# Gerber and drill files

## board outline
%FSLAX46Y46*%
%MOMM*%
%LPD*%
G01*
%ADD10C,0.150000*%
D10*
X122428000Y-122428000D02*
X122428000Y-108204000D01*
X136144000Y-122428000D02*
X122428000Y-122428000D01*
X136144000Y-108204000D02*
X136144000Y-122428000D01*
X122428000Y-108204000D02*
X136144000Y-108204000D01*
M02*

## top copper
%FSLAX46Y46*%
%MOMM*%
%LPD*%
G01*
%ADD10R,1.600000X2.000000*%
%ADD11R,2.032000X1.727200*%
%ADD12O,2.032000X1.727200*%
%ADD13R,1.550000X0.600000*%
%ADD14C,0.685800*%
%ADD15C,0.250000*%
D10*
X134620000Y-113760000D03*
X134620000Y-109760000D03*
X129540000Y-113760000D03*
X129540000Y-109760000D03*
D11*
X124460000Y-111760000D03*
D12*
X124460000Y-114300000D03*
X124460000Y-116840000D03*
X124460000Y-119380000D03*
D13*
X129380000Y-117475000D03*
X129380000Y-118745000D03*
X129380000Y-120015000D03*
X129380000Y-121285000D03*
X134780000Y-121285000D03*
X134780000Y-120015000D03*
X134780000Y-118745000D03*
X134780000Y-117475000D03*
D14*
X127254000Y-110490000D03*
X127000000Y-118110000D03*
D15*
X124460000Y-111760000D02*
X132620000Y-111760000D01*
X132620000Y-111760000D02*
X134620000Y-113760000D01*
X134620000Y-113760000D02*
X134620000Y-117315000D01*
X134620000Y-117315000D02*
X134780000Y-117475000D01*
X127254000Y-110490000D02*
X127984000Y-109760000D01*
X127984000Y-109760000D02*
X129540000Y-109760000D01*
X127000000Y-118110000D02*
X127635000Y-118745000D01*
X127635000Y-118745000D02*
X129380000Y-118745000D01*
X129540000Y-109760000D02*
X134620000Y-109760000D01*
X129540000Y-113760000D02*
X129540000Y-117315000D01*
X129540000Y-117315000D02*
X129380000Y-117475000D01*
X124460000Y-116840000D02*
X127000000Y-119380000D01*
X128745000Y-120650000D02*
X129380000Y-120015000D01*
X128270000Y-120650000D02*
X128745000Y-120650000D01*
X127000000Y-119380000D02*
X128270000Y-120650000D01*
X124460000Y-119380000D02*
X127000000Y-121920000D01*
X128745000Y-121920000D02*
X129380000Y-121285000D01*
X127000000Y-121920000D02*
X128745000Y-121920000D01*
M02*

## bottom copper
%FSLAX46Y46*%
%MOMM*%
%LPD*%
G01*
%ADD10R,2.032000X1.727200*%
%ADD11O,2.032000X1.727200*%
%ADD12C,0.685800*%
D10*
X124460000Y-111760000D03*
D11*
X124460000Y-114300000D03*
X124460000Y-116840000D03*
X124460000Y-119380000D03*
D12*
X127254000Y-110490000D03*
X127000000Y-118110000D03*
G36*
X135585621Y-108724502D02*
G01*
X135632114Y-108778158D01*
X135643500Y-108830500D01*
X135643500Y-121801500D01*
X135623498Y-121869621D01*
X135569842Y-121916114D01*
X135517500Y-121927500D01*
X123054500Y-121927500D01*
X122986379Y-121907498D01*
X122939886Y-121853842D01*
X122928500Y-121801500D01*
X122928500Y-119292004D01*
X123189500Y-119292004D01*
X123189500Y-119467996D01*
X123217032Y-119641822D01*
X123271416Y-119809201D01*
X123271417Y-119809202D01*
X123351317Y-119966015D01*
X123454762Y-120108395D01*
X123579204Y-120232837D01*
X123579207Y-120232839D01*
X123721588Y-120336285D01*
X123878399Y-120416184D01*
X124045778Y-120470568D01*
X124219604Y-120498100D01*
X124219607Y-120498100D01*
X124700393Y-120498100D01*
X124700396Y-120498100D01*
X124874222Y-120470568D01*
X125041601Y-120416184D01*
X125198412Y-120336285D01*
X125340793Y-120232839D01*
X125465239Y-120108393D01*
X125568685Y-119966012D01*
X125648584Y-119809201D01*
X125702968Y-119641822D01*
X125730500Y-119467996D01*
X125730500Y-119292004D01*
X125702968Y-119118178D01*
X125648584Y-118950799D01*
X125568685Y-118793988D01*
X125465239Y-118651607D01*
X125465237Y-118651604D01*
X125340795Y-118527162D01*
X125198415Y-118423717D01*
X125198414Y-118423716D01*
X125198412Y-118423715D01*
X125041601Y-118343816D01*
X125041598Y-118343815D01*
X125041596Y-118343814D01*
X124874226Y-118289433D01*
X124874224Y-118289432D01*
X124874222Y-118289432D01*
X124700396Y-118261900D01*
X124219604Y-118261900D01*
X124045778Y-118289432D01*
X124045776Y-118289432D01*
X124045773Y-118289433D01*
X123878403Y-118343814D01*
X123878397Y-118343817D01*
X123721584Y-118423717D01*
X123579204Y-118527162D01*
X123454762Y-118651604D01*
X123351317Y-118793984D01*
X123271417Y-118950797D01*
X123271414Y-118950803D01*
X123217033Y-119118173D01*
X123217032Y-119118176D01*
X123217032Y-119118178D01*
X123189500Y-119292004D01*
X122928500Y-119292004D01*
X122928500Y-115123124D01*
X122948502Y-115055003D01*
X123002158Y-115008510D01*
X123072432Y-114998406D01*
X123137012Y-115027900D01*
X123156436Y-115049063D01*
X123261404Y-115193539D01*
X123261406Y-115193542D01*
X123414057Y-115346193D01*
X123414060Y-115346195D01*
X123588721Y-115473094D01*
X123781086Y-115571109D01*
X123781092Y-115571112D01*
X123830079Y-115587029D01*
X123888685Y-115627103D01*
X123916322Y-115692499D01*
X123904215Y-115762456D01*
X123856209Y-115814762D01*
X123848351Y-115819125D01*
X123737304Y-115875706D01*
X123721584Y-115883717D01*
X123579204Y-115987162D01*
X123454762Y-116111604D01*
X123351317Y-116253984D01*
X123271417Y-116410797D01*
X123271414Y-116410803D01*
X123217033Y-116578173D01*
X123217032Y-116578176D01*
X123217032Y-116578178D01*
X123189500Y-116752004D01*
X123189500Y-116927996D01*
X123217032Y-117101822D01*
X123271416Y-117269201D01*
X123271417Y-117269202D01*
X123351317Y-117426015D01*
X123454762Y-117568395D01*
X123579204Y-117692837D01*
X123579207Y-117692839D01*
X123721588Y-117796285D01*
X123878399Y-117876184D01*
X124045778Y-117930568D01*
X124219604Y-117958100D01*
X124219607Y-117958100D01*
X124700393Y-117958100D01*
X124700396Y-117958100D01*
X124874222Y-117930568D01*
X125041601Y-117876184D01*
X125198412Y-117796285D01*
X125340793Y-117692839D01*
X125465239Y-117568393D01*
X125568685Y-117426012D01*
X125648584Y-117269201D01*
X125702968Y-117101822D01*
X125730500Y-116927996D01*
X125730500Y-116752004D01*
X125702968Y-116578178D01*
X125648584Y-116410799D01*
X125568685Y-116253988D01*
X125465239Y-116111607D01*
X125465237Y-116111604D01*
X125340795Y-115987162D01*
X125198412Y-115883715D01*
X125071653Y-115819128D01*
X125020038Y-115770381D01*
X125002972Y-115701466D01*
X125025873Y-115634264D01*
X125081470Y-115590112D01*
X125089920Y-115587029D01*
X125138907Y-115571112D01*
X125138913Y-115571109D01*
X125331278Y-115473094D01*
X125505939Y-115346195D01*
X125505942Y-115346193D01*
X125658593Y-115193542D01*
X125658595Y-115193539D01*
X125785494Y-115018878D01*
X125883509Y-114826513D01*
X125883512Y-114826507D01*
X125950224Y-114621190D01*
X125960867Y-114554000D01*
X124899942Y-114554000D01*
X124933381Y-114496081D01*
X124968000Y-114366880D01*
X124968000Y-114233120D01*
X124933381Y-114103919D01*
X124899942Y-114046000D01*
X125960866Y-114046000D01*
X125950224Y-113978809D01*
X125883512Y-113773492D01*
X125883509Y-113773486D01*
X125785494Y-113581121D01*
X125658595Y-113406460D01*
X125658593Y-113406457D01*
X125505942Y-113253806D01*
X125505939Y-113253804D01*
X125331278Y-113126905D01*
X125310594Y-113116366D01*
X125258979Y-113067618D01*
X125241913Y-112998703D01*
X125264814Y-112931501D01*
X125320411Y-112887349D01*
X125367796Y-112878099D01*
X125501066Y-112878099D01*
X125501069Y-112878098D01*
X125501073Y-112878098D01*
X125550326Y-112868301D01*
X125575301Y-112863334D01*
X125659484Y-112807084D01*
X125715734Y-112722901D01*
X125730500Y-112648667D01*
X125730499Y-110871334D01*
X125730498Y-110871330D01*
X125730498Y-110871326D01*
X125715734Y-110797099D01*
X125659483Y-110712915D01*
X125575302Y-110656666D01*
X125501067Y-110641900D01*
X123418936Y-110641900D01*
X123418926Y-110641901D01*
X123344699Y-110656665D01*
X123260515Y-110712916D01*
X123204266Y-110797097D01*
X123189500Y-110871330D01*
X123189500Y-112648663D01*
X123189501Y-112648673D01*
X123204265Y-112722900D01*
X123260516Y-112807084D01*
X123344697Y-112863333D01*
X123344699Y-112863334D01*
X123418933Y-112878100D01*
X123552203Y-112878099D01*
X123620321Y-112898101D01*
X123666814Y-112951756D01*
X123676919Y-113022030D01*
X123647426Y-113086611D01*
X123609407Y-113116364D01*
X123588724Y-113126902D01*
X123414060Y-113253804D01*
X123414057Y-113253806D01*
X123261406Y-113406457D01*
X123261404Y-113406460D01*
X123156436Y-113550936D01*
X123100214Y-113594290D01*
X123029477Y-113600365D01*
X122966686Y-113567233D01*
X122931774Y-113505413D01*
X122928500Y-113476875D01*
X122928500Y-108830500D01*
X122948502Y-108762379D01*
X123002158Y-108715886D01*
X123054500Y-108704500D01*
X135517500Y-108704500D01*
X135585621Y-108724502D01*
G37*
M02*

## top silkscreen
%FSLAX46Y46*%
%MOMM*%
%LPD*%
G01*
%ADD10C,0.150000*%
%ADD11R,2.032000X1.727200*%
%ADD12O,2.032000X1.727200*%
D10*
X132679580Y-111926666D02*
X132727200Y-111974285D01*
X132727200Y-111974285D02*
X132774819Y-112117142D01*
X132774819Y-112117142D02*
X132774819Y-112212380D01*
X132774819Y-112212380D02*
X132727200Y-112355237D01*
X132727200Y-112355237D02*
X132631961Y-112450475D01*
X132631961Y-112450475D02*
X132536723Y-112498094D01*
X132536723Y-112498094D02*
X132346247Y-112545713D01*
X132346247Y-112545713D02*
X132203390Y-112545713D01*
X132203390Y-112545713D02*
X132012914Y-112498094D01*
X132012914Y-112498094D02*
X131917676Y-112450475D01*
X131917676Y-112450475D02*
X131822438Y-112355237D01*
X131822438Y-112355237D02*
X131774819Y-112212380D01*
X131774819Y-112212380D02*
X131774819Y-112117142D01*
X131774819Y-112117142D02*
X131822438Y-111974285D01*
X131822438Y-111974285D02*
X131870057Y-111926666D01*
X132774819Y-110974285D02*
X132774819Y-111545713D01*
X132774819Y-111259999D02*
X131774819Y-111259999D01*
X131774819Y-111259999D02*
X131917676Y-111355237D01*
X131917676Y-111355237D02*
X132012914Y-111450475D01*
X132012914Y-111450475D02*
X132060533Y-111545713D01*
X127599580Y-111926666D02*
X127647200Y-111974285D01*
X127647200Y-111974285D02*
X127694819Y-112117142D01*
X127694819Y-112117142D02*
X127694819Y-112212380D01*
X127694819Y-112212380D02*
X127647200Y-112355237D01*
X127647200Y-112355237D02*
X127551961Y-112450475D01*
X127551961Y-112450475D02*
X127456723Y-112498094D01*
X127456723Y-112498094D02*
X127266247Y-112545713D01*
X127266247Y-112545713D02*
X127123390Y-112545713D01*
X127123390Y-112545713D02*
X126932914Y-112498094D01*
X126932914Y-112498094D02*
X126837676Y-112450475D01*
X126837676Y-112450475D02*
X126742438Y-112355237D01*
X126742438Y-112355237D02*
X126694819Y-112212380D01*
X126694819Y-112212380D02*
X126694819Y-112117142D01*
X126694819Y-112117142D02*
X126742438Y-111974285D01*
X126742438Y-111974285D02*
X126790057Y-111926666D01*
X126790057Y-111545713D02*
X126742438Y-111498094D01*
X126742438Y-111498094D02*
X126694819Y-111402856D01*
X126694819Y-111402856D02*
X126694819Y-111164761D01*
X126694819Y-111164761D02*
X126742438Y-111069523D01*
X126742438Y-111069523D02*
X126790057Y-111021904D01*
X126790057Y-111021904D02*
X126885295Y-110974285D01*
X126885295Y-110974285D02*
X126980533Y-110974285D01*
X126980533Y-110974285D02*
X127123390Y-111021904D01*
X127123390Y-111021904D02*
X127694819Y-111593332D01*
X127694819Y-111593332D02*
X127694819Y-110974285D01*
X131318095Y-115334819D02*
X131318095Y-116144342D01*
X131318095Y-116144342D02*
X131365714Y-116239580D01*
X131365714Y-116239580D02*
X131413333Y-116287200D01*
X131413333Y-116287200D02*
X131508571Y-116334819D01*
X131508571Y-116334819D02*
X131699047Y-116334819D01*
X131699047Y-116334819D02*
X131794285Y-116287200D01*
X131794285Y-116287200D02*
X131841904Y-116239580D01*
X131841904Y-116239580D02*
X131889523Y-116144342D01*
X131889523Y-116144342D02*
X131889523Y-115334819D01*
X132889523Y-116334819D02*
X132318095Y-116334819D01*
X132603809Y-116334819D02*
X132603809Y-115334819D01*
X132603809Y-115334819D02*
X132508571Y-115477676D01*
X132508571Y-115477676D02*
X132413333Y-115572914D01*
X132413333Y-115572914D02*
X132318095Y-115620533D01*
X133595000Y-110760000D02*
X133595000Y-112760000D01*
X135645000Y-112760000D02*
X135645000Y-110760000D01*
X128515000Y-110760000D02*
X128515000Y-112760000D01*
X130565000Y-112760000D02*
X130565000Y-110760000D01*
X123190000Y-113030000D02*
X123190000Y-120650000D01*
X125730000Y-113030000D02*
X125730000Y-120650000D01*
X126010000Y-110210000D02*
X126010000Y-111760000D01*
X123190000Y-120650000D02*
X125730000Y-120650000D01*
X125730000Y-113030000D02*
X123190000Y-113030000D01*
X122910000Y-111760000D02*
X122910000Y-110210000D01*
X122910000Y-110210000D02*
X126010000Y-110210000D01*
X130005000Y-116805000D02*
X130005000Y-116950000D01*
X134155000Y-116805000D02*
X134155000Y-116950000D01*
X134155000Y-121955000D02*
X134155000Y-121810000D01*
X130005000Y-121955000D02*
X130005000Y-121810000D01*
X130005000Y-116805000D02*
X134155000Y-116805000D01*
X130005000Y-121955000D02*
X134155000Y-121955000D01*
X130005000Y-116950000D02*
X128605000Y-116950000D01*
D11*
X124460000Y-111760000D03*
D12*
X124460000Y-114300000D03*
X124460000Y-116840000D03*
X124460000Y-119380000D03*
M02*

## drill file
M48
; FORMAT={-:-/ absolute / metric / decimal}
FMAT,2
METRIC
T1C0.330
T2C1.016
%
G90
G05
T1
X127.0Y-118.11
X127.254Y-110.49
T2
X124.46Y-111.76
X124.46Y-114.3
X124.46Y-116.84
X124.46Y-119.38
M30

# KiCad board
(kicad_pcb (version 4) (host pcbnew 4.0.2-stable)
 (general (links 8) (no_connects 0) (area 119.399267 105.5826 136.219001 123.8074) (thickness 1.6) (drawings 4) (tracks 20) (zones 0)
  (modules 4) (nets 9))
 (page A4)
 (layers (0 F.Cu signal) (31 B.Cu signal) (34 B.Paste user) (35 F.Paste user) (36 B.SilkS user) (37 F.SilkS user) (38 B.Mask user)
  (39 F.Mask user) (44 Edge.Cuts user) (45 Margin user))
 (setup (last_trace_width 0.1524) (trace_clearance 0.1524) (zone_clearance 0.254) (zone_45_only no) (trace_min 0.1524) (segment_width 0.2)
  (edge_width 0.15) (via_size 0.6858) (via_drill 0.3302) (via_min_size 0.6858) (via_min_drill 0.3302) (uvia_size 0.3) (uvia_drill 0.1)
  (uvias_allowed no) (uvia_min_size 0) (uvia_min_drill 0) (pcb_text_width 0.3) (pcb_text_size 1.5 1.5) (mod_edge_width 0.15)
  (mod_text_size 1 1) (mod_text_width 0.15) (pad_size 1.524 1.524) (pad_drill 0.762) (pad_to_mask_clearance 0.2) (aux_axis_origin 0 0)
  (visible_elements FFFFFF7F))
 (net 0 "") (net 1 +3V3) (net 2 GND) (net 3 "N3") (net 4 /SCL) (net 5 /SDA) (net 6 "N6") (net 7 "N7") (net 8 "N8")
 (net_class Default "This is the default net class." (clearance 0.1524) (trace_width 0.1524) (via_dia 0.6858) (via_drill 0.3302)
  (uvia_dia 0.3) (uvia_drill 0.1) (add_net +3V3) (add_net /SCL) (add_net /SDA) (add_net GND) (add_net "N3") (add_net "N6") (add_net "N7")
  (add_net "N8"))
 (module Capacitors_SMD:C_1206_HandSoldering (layer F.Cu) (at 134.62 111.76 90)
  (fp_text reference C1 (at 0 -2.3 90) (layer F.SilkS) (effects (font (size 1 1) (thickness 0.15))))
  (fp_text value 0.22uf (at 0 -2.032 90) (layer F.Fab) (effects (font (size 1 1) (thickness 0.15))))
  (fp_line (start 1 -1.025) (end -1 -1.025) (layer F.SilkS) (width 0.15))
  (fp_line (start -1 1.025) (end 1 1.025) (layer F.SilkS) (width 0.15))
  (pad 1 smd rect (at -2 0 90) (size 2 1.6) (layers F.Cu F.Paste F.Mask) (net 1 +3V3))
  (pad 2 smd rect (at 2 0 90) (size 2 1.6) (layers F.Cu F.Paste F.Mask) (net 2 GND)))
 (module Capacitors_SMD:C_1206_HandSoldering (layer F.Cu) (at 129.54 111.76 90)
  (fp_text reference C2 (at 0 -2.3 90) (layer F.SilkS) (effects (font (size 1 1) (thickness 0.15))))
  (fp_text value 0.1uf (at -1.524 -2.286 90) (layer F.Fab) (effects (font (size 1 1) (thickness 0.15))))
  (fp_line (start 1 -1.025) (end -1 -1.025) (layer F.SilkS) (width 0.15))
  (fp_line (start -1 1.025) (end 1 1.025) (layer F.SilkS) (width 0.15))
  (pad 1 smd rect (at -2 0 90) (size 2 1.6) (layers F.Cu F.Paste F.Mask) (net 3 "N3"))
  (pad 2 smd rect (at 2 0 90) (size 2 1.6) (layers F.Cu F.Paste F.Mask) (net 2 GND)))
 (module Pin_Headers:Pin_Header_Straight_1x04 (layer F.Cu) (at 124.46 111.76)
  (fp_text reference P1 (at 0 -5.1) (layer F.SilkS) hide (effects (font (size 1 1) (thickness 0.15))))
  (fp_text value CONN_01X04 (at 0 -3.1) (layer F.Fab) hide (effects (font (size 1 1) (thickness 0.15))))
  (fp_line (start -1.27 1.27) (end -1.27 8.89) (layer F.SilkS) (width 0.15))
  (fp_line (start 1.27 1.27) (end 1.27 8.89) (layer F.SilkS) (width 0.15))
  (fp_line (start 1.55 -1.55) (end 1.55 0) (layer F.SilkS) (width 0.15))
  (fp_line (start -1.27 8.89) (end 1.27 8.89) (layer F.SilkS) (width 0.15))
  (fp_line (start 1.27 1.27) (end -1.27 1.27) (layer F.SilkS) (width 0.15))
  (fp_line (start -1.55 0) (end -1.55 -1.55) (layer F.SilkS) (width 0.15))
  (fp_line (start -1.55 -1.55) (end 1.55 -1.55) (layer F.SilkS) (width 0.15))
  (pad 1 thru_hole rect (at 0 0) (size 2.032 1.7272) (drill 1.016) (layers *.Cu *.Mask F.SilkS) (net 1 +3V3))
  (pad 2 thru_hole oval (at 0 2.54) (size 2.032 1.7272) (drill 1.016) (layers *.Cu *.Mask F.SilkS) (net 2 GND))
  (pad 3 thru_hole oval (at 0 5.08) (size 2.032 1.7272) (drill 1.016) (layers *.Cu *.Mask F.SilkS) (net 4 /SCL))
  (pad 4 thru_hole oval (at 0 7.62) (size 2.032 1.7272) (drill 1.016) (layers *.Cu *.Mask F.SilkS) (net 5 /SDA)))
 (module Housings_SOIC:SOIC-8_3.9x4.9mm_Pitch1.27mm (layer F.Cu) (at 132.08 119.38)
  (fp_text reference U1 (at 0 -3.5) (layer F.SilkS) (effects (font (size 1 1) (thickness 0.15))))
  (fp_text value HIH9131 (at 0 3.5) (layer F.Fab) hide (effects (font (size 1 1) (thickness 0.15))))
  (fp_line (start -2.075 -2.575) (end -2.075 -2.43) (layer F.SilkS) (width 0.15))
  (fp_line (start 2.075 -2.575) (end 2.075 -2.43) (layer F.SilkS) (width 0.15))
  (fp_line (start 2.075 2.575) (end 2.075 2.43) (layer F.SilkS) (width 0.15))
  (fp_line (start -2.075 2.575) (end -2.075 2.43) (layer F.SilkS) (width 0.15))
  (fp_line (start -2.075 -2.575) (end 2.075 -2.575) (layer F.SilkS) (width 0.15))
  (fp_line (start -2.075 2.575) (end 2.075 2.575) (layer F.SilkS) (width 0.15))
  (fp_line (start -2.075 -2.43) (end -3.475 -2.43) (layer F.SilkS) (width 0.15))
  (pad 1 smd rect (at -2.7 -1.905) (size 1.55 0.6) (layers F.Cu F.Paste F.Mask) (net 3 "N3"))
  (pad 2 smd rect (at -2.7 -0.635) (size 1.55 0.6) (layers F.Cu F.Paste F.Mask) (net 2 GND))
  (pad 3 smd rect (at -2.7 0.635) (size 1.55 0.6) (layers F.Cu F.Paste F.Mask) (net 4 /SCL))
  (pad 4 smd rect (at -2.7 1.905) (size 1.55 0.6) (layers F.Cu F.Paste F.Mask) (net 5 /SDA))
  (pad 5 smd rect (at 2.7 1.905) (size 1.55 0.6) (layers F.Cu F.Paste F.Mask) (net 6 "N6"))
  (pad 6 smd rect (at 2.7 0.635) (size 1.55 0.6) (layers F.Cu F.Paste F.Mask) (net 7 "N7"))
  (pad 7 smd rect (at 2.7 -0.635) (size 1.55 0.6) (layers F.Cu F.Paste F.Mask) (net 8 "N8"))
  (pad 8 smd rect (at 2.7 -1.905) (size 1.55 0.6) (layers F.Cu F.Paste F.Mask) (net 1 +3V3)))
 (gr_line (start 122.428 122.428) (end 122.428 108.204) (angle 90) (layer Edge.Cuts) (width 0.15))
 (gr_line (start 136.144 122.428) (end 122.428 122.428) (angle 90) (layer Edge.Cuts) (width 0.15))
 (gr_line (start 136.144 108.204) (end 136.144 122.428) (angle 90) (layer Edge.Cuts) (width 0.15))
 (gr_line (start 122.428 108.204) (end 136.144 108.204) (angle 90) (layer Edge.Cuts) (width 0.15))
 (segment (start 124.46 111.76) (end 132.62 111.76) (width 0.25) (layer F.Cu) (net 1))
 (segment (start 132.62 111.76) (end 134.62 113.76) (width 0.25) (layer F.Cu) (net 1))
 (segment (start 134.62 113.76) (end 134.62 117.315) (width 0.25) (layer F.Cu) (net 1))
 (segment (start 134.62 117.315) (end 134.78 117.475) (width 0.25) (layer F.Cu) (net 1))
 (via (at 127.254 110.49) (size 0.6858) (drill 0.3302) (layers F.Cu B.Cu) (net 2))
 (segment (start 127.254 110.49) (end 127.984 109.76) (width 0.25) (layer F.Cu) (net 2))
 (segment (start 127.984 109.76) (end 129.54 109.76) (width 0.25) (layer F.Cu) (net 2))
 (via (at 127 118.11) (size 0.6858) (drill 0.3302) (layers F.Cu B.Cu) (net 2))
 (segment (start 127 118.11) (end 127.635 118.745) (width 0.25) (layer F.Cu) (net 2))
 (segment (start 127.635 118.745) (end 129.38 118.745) (width 0.25) (layer F.Cu) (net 2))
 (segment (start 129.54 109.76) (end 134.62 109.76) (width 0.25) (layer F.Cu) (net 2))
 (segment (start 129.54 113.76) (end 129.54 117.315) (width 0.25) (layer F.Cu) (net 3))
 (segment (start 129.54 117.315) (end 129.38 117.475) (width 0.25) (layer F.Cu) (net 3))
 (segment (start 124.46 116.84) (end 127 119.38) (width 0.25) (layer F.Cu) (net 4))
 (segment (start 128.745 120.65) (end 129.38 120.015) (width 0.25) (layer F.Cu) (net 4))
 (segment (start 128.27 120.65) (end 128.745 120.65) (width 0.25) (layer F.Cu) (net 4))
 (segment (start 127 119.38) (end 128.27 120.65) (width 0.25) (layer F.Cu) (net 4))
 (segment (start 124.46 119.38) (end 127 121.92) (width 0.25) (layer F.Cu) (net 5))
 (segment (start 128.745 121.92) (end 129.38 121.285) (width 0.25) (layer F.Cu) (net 5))
 (segment (start 127 121.92) (end 128.745 121.92) (width 0.25) (layer F.Cu) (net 5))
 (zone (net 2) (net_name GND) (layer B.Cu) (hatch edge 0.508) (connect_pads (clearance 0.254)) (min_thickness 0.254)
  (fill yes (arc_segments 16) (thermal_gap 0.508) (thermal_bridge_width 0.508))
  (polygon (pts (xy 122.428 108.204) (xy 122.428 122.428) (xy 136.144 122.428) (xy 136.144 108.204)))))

